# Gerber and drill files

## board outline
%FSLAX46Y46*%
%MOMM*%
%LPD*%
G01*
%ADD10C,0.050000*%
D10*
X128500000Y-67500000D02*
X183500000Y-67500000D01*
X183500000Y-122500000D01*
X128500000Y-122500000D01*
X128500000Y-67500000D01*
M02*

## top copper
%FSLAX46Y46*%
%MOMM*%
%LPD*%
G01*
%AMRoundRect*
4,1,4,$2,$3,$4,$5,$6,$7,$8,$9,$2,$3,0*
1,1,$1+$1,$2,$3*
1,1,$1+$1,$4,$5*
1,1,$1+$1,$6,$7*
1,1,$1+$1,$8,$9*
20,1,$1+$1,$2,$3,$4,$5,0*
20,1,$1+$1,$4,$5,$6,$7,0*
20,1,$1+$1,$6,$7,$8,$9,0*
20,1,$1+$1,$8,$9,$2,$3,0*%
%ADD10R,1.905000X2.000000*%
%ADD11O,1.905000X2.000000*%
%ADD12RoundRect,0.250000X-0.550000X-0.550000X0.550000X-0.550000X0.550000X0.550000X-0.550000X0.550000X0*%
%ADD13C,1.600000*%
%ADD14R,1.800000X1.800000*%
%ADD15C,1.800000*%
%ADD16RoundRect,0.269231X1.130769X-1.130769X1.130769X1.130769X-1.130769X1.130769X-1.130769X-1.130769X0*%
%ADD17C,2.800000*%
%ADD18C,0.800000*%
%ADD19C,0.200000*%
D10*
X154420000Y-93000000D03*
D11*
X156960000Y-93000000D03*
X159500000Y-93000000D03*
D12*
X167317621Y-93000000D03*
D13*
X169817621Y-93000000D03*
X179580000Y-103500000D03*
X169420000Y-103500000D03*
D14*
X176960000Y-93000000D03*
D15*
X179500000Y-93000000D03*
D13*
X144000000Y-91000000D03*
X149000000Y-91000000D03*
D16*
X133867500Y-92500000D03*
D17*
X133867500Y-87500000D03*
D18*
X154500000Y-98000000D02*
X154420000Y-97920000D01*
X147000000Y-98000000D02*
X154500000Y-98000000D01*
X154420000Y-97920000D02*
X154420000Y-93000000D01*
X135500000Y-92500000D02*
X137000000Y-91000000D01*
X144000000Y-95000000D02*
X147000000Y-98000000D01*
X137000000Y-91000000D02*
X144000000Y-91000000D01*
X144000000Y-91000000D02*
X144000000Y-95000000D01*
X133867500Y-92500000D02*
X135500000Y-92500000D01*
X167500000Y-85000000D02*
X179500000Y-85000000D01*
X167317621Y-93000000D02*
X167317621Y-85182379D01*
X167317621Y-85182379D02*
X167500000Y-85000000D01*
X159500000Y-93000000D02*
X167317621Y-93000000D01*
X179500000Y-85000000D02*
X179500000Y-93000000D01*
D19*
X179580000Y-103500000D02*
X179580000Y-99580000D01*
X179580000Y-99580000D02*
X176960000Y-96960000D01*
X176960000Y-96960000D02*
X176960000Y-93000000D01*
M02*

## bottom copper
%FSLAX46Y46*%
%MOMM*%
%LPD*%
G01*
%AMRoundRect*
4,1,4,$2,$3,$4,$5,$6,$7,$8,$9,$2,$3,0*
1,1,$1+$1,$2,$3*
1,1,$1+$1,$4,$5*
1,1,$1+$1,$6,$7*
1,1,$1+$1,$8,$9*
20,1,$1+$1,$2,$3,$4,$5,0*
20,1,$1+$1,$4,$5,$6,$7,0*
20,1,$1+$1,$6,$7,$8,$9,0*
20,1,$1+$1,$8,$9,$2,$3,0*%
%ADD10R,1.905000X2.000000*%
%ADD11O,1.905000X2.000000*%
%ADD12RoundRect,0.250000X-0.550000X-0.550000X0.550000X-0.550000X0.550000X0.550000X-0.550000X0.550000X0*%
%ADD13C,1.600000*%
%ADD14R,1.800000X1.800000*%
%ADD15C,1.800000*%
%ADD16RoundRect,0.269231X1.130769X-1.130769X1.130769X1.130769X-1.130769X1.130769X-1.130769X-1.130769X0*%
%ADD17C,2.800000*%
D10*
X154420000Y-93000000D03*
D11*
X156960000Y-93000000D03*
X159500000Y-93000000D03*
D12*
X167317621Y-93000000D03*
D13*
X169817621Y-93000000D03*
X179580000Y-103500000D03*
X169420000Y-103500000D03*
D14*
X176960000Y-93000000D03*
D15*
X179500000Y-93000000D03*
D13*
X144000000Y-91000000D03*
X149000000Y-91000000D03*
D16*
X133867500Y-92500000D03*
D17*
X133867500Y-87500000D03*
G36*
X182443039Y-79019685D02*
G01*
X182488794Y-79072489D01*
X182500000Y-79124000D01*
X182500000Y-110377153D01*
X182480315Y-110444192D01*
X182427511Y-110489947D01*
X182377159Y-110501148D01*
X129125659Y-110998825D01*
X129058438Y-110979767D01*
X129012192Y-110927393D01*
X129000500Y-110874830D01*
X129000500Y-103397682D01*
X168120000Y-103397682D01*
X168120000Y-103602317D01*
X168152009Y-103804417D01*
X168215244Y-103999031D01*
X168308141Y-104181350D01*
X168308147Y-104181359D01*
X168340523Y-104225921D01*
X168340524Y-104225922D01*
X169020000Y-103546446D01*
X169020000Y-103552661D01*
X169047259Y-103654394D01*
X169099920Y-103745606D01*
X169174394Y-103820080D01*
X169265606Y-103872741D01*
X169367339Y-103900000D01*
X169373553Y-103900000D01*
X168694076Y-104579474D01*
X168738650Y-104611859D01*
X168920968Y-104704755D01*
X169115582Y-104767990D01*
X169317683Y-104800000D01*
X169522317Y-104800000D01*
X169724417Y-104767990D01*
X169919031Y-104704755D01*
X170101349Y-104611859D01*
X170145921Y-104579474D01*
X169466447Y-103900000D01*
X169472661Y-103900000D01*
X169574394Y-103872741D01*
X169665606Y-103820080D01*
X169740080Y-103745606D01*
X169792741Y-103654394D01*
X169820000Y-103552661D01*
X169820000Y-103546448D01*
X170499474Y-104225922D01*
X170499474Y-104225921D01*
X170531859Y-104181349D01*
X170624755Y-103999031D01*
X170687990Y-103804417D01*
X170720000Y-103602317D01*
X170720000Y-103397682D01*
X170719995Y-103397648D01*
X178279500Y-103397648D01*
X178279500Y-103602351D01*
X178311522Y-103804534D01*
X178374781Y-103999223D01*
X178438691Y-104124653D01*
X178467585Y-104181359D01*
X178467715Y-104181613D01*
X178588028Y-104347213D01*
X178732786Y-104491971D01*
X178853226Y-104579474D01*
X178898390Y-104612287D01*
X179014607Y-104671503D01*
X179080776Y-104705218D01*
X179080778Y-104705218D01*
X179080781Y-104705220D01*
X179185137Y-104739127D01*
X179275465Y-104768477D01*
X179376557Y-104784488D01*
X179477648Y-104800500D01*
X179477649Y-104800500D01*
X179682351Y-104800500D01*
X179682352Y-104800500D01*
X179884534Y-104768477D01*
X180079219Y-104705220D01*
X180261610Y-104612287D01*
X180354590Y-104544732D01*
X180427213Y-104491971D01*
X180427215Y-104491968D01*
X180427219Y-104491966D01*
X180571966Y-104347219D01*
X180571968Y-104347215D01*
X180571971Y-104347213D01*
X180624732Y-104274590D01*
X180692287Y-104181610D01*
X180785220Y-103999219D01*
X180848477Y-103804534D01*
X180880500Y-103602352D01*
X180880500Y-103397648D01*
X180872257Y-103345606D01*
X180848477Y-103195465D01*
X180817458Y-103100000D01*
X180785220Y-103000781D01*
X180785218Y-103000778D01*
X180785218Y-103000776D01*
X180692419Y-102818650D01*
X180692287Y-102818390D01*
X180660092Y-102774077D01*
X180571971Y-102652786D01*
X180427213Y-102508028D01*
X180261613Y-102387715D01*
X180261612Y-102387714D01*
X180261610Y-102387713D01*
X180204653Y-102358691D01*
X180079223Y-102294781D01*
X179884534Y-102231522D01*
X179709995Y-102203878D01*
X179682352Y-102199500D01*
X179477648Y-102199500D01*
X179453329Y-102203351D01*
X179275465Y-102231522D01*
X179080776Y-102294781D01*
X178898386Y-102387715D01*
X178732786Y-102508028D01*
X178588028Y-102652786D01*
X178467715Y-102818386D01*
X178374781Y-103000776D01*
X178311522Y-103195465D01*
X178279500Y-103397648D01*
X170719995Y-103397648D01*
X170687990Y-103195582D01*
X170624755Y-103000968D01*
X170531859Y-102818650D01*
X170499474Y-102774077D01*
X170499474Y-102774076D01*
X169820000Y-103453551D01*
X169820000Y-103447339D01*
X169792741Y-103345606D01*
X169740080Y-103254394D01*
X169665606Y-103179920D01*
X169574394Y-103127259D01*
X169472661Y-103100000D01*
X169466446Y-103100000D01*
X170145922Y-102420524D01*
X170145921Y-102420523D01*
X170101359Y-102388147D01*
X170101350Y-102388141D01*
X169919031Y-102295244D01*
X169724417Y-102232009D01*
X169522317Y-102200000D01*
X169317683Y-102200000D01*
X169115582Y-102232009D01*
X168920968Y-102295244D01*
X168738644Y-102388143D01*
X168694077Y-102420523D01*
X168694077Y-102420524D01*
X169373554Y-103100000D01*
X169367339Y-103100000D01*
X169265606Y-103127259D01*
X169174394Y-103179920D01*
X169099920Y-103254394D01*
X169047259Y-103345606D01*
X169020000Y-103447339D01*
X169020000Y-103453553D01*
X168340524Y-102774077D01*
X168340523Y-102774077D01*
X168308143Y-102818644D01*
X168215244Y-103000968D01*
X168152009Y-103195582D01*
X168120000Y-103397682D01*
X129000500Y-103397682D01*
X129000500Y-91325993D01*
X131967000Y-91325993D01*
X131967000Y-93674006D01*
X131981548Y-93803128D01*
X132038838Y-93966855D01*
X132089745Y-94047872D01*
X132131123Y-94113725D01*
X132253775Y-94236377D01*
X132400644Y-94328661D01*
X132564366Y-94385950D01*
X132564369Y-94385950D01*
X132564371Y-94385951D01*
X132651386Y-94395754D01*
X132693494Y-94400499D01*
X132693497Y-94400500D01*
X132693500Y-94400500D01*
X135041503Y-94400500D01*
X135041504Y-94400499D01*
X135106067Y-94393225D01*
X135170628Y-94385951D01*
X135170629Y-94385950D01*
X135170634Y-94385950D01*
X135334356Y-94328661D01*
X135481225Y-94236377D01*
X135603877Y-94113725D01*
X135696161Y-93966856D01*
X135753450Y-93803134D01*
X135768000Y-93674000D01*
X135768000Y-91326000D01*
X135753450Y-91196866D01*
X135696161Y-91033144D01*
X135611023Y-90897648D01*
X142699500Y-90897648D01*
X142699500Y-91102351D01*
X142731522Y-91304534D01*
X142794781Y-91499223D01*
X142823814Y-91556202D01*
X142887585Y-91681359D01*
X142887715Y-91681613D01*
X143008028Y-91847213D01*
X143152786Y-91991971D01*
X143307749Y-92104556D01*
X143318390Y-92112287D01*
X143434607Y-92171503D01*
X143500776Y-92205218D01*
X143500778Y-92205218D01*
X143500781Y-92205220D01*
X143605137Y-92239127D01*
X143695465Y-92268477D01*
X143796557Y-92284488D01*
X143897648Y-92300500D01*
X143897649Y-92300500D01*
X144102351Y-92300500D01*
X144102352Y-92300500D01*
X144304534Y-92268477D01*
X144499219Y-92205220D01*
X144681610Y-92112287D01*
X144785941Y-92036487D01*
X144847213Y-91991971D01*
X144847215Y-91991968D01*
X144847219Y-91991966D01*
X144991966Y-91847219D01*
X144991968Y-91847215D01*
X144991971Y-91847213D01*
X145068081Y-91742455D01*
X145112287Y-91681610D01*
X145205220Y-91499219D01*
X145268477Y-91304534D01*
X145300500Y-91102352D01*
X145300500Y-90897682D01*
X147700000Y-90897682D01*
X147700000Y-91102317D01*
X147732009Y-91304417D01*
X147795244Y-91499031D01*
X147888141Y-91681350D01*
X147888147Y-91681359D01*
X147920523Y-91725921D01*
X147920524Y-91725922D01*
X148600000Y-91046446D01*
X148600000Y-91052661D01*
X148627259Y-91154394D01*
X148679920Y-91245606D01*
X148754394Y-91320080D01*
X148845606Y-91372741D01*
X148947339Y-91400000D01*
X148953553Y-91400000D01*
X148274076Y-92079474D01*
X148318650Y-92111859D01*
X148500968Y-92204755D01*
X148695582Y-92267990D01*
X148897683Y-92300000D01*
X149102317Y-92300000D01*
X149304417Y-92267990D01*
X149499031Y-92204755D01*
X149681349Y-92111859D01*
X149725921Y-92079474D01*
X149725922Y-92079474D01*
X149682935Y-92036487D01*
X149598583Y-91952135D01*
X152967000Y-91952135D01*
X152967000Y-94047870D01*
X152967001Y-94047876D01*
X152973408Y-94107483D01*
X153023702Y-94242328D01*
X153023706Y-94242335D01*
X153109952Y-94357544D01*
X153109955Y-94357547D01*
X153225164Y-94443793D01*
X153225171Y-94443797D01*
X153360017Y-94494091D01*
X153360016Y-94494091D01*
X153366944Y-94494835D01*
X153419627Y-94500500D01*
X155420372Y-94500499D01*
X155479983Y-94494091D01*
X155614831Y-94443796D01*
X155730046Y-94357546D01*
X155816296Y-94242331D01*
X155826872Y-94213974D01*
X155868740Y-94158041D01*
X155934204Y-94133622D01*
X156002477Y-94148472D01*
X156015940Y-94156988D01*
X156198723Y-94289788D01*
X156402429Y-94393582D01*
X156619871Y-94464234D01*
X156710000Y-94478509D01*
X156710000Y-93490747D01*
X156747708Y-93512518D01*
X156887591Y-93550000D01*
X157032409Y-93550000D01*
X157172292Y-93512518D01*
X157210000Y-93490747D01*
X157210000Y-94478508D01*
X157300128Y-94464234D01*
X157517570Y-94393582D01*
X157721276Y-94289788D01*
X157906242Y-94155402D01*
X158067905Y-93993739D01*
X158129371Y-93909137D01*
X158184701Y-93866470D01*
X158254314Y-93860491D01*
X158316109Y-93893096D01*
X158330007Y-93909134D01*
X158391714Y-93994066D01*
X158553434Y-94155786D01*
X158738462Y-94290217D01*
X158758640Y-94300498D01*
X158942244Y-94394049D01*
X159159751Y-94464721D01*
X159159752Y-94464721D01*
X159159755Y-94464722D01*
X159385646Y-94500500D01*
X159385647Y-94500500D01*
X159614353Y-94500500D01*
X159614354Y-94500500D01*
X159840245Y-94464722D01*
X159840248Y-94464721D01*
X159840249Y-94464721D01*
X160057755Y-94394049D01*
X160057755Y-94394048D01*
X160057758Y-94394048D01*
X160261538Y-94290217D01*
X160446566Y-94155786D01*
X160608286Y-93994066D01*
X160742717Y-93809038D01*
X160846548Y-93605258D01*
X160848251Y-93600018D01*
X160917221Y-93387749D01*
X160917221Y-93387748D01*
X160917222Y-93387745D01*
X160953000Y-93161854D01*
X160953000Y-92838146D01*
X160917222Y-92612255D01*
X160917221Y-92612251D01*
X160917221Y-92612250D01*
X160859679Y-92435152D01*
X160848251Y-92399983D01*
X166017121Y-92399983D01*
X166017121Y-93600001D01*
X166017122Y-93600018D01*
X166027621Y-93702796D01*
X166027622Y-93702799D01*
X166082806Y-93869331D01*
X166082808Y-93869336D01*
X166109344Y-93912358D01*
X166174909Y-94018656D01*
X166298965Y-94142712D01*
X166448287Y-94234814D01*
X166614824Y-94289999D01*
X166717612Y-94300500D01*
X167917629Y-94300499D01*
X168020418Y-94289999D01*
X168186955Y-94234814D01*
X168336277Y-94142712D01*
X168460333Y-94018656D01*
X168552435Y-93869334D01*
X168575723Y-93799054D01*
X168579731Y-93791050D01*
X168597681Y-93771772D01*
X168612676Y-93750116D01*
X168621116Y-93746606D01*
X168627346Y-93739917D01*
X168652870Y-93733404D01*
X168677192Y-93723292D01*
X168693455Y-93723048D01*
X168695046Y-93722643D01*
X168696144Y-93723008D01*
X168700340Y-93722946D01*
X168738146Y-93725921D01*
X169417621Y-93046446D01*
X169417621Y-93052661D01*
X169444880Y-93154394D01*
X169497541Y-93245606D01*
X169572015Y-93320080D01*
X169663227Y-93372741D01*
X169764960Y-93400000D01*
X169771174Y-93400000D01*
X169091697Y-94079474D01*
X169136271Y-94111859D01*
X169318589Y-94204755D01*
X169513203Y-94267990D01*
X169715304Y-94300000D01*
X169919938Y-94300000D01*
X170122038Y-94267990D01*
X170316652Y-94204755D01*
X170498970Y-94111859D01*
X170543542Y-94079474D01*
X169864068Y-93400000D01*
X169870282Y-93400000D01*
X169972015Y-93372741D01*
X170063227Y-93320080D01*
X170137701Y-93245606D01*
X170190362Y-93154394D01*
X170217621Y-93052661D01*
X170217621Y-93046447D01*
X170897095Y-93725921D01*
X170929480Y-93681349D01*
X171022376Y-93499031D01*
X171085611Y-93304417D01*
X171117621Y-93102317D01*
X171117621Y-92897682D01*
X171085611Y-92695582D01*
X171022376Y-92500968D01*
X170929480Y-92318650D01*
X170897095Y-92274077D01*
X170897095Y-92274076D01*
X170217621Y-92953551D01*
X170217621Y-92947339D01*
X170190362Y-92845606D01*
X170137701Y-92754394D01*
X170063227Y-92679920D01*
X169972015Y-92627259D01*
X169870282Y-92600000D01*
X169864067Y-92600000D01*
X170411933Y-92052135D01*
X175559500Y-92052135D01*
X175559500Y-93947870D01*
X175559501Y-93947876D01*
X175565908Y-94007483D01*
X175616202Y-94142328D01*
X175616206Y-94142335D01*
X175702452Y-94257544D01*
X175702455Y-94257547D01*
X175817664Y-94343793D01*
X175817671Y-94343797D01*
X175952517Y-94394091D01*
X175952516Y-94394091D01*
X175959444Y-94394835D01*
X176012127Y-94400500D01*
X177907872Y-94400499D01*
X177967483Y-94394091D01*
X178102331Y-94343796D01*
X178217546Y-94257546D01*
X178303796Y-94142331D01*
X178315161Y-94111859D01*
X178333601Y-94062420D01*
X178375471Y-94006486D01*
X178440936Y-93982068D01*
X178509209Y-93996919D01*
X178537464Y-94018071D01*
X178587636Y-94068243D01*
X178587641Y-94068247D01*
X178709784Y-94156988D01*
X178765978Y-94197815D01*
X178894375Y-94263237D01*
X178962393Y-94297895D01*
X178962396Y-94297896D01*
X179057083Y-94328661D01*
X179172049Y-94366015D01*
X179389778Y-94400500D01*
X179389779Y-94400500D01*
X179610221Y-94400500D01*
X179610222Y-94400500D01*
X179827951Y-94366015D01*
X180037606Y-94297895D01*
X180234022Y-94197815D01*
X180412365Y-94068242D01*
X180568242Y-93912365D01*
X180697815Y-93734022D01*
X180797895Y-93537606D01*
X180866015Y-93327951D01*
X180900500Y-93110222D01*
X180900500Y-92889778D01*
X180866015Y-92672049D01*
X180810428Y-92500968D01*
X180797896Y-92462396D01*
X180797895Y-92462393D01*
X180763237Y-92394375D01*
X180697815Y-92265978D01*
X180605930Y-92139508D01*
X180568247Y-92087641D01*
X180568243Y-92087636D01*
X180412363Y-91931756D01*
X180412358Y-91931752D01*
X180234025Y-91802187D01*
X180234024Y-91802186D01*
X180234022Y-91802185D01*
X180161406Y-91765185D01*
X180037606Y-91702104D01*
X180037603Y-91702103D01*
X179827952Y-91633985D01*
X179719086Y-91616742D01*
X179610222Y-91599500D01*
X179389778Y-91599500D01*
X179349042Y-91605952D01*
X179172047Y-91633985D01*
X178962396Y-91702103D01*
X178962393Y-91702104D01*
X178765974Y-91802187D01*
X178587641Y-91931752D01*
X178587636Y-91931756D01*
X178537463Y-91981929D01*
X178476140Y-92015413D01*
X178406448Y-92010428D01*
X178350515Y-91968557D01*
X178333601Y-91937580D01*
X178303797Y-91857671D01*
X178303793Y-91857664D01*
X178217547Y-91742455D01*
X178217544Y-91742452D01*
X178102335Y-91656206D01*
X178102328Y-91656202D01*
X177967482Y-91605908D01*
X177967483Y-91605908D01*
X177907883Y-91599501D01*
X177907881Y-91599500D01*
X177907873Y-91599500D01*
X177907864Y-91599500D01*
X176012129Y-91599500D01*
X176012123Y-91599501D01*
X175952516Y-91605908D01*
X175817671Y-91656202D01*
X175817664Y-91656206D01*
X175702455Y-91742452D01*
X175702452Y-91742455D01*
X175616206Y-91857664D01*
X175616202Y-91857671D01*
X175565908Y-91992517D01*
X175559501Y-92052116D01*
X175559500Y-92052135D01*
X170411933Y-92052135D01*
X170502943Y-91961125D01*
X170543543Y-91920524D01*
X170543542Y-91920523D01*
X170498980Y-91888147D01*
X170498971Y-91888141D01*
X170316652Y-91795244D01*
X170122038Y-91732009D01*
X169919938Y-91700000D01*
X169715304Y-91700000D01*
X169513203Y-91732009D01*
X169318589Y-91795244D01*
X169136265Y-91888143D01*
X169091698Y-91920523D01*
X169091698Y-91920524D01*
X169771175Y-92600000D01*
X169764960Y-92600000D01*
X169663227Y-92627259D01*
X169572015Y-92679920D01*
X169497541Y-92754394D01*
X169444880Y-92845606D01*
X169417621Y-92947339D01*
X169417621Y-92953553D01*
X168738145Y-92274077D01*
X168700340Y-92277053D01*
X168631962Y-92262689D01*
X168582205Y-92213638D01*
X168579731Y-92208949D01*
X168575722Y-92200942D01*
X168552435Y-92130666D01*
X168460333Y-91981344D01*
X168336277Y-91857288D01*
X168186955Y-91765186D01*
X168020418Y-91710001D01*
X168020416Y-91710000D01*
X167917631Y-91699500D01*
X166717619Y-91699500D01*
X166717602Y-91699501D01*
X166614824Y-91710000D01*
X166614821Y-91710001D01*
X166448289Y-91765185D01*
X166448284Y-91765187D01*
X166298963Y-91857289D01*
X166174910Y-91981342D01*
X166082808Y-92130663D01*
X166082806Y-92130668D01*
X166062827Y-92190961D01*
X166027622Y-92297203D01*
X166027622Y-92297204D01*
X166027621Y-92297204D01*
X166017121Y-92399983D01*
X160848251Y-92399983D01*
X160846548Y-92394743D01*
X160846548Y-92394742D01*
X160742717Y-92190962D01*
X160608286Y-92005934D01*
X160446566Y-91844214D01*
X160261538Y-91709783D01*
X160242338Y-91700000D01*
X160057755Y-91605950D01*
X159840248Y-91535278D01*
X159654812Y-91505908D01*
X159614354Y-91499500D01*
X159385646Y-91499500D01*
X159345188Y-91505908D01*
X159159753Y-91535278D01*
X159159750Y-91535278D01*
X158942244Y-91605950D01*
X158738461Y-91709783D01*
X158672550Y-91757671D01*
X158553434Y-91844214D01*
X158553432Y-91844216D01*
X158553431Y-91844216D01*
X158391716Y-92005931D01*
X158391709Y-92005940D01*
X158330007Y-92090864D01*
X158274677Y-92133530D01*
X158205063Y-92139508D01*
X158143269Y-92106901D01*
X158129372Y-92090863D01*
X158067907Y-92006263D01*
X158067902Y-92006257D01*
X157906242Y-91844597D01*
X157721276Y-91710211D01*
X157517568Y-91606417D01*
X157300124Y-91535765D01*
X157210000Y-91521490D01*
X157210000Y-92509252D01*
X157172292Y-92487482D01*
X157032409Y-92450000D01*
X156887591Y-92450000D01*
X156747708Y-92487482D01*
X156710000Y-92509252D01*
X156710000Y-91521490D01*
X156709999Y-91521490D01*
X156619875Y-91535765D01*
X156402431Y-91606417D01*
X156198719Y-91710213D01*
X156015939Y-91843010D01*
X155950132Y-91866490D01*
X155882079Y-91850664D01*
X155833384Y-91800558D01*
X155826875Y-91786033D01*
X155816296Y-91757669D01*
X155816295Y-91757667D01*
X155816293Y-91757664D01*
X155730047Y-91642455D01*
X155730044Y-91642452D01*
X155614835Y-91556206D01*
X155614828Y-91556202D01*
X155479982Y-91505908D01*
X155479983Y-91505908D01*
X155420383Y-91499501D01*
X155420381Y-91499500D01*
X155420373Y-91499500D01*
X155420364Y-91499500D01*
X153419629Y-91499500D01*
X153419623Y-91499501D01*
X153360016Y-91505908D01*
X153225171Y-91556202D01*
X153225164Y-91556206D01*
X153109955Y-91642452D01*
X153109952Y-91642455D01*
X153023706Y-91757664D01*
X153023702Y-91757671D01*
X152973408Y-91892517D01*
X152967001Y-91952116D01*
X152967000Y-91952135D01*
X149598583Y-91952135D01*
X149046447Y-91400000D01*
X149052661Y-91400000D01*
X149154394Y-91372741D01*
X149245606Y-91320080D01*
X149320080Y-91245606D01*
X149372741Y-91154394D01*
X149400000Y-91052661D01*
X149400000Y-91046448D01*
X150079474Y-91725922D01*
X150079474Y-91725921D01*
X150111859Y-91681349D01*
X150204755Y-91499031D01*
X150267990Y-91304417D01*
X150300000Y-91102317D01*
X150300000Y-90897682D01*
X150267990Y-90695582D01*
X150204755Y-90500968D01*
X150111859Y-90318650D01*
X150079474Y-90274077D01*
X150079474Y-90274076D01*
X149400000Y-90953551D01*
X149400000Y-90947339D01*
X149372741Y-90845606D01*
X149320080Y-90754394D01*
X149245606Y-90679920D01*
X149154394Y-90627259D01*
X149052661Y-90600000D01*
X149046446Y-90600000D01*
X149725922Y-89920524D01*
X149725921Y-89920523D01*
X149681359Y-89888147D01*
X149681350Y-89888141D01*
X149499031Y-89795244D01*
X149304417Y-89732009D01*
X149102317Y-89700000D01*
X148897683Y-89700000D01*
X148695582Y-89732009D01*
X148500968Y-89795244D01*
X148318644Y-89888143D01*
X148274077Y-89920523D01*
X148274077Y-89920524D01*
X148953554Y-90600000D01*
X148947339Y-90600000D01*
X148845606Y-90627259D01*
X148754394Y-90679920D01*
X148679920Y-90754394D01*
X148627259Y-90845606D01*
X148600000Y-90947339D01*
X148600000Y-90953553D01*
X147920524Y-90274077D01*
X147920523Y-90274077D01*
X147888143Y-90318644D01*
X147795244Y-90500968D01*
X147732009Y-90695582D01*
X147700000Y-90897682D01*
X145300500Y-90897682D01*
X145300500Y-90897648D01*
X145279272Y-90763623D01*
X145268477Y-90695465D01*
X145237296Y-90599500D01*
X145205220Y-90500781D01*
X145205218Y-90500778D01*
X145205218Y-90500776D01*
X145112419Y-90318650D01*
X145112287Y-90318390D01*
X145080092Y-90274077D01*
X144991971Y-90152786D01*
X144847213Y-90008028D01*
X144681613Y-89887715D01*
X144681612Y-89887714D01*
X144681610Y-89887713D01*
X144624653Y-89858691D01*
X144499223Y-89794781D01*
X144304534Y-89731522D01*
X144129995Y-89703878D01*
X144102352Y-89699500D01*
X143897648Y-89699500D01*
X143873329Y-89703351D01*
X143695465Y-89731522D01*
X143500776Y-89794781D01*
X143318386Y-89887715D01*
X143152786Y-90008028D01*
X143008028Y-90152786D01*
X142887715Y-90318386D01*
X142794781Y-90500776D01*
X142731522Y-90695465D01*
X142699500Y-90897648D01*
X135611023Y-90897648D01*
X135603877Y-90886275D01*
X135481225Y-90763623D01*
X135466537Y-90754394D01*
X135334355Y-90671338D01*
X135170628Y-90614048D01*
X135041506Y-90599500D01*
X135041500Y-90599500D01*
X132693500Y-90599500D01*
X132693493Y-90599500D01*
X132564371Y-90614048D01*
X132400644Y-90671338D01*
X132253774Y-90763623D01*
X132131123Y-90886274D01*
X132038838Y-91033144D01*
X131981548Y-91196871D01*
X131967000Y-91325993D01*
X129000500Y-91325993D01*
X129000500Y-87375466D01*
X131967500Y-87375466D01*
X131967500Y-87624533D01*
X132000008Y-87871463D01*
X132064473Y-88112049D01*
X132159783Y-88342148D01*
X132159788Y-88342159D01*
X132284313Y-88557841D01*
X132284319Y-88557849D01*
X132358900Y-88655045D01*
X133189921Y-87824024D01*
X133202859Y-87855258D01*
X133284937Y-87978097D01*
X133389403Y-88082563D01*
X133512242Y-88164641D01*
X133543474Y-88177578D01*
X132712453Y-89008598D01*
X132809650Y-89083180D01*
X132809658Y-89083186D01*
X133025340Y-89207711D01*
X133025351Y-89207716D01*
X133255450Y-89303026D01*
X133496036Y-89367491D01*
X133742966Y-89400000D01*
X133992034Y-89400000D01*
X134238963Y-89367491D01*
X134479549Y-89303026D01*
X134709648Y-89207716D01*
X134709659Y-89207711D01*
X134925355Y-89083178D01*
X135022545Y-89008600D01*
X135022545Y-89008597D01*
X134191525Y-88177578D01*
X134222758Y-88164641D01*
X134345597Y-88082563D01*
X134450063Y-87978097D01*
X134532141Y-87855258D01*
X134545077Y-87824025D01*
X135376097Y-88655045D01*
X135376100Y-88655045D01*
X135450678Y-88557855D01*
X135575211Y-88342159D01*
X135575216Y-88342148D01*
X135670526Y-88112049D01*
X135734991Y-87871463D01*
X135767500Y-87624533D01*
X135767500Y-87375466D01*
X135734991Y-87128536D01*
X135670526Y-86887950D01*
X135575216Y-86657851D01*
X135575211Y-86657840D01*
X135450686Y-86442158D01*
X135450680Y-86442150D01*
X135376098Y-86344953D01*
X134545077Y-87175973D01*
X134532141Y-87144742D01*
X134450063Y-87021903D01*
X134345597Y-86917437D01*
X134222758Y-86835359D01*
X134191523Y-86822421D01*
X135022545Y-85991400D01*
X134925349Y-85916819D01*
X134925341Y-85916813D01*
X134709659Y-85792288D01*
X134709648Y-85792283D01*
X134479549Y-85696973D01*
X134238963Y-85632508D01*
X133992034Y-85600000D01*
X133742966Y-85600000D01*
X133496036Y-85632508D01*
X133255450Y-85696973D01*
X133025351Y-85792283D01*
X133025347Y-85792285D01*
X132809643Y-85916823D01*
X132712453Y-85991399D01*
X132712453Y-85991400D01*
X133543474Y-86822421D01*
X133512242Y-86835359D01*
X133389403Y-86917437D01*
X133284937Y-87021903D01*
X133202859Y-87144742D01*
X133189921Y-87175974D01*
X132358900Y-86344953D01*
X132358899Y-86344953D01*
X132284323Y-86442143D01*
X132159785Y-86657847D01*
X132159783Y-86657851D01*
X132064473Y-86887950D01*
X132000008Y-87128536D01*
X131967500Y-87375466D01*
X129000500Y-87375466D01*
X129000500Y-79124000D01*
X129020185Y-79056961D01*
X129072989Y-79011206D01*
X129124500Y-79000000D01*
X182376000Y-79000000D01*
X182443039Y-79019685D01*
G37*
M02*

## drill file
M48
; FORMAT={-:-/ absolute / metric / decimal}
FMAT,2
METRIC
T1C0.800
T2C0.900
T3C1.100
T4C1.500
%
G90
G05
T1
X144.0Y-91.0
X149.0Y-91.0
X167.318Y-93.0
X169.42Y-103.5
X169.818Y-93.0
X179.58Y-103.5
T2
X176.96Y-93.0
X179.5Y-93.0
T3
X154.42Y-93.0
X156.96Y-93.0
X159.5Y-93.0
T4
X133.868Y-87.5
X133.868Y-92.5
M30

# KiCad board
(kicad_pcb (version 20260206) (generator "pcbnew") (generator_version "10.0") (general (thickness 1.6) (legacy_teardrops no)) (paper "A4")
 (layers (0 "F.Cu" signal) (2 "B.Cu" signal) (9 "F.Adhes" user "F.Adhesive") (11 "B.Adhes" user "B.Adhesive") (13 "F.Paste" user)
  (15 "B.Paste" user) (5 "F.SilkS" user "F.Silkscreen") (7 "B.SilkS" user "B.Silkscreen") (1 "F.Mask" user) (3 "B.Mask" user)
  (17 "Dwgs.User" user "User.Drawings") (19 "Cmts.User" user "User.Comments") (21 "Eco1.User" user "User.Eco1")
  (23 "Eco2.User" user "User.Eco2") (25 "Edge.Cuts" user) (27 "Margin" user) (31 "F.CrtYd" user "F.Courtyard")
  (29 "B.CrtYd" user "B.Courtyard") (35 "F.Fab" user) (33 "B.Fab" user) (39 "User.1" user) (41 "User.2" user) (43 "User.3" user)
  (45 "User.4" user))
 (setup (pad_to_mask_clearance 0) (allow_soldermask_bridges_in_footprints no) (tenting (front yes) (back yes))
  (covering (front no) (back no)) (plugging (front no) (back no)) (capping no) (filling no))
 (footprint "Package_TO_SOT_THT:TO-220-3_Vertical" (layer "F.Cu") (at 154.42 93)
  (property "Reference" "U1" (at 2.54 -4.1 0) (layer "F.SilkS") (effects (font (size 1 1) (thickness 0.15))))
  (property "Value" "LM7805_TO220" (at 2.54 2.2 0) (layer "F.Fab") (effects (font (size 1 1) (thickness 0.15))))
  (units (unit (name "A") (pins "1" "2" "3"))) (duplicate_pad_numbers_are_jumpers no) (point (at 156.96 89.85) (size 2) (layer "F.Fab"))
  (pad "1" thru_hole rect (at 0 0) (size 1.905 2) (drill 1.1) (layers "*.Cu" "*.Mask") (remove_unused_layers no) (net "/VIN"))
  (pad "2" thru_hole oval (at 2.54 0) (size 1.905 2) (drill 1.1) (layers "*.Cu" "*.Mask") (remove_unused_layers no) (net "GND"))
  (pad "3" thru_hole oval (at 5.08 0) (size 1.905 2) (drill 1.1) (layers "*.Cu" "*.Mask") (remove_unused_layers no) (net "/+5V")))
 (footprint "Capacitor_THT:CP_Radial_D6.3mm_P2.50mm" (layer "F.Cu") (at 167.317621 93)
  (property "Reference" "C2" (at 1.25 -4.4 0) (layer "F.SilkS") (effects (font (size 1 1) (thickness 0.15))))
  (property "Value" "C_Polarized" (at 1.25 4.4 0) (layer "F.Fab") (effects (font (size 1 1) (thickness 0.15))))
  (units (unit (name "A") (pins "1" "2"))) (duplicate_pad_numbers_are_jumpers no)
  (pad "1" thru_hole roundrect (at 0 0) (size 1.6 1.6) (drill 0.8) (layers "*.Cu" "*.Mask") (remove_unused_layers no)
   (roundrect_rratio 0.15625) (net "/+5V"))
  (pad "2" thru_hole circle (at 2.5 0) (size 1.6 1.6) (drill 0.8) (layers "*.Cu" "*.Mask") (remove_unused_layers no) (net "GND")))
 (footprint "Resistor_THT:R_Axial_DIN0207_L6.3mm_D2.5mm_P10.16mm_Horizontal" (layer "F.Cu") (at 179.58 103.5 180)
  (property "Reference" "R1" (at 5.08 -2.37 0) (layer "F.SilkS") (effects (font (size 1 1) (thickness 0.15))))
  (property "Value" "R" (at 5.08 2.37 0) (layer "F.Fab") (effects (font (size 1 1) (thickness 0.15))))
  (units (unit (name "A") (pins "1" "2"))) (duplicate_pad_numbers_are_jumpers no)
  (pad "1" thru_hole circle (at 0 0 180) (size 1.6 1.6) (drill 0.8) (layers "*.Cu" "*.Mask") (remove_unused_layers no) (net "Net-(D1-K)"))
  (pad "2" thru_hole circle (at 10.16 0 180) (size 1.6 1.6) (drill 0.8) (layers "*.Cu" "*.Mask") (remove_unused_layers no) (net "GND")))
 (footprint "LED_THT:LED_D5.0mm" (layer "F.Cu") (at 176.96 93)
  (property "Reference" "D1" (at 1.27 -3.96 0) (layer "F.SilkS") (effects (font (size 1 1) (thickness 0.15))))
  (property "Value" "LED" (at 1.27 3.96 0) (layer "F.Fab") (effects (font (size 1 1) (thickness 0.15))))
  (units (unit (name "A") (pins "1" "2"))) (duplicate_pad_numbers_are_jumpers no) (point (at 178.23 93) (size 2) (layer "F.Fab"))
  (pad "1" thru_hole rect (at 0 0) (size 1.8 1.8) (drill 0.9) (layers "*.Cu" "*.Mask") (remove_unused_layers no) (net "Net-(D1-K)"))
  (pad "2" thru_hole circle (at 2.54 0) (size 1.8 1.8) (drill 0.9) (layers "*.Cu" "*.Mask") (remove_unused_layers no) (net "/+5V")))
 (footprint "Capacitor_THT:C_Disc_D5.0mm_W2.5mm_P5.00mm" (layer "F.Cu") (at 144 91)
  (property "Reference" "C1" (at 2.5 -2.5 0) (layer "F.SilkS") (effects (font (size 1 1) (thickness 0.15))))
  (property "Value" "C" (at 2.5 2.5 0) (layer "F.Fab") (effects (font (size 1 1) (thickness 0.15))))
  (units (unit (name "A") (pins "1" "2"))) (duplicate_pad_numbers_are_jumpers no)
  (pad "1" thru_hole circle (at 0 0) (size 1.6 1.6) (drill 0.8) (layers "*.Cu" "*.Mask") (remove_unused_layers no) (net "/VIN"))
  (pad "2" thru_hole circle (at 5 0) (size 1.6 1.6) (drill 0.8) (layers "*.Cu" "*.Mask") (remove_unused_layers no) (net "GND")))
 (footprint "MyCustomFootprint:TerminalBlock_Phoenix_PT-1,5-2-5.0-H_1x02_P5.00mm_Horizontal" (layer "F.Cu") (at 133.8675 92.5 90)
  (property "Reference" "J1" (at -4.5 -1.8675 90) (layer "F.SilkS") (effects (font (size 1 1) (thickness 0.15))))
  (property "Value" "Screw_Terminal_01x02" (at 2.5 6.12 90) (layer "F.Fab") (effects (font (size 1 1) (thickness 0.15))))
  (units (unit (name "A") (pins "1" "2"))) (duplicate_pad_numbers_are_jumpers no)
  (pad "1" thru_hole roundrect (at 0 0 90) (size 2.8 2.8) (drill 1.5) (layers "*.Cu" "*.Mask") (remove_unused_layers no)
   (roundrect_rratio 0.096154) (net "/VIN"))
  (pad "2" thru_hole circle (at 5 0 90) (size 2.8 2.8) (drill 1.5) (layers "*.Cu" "*.Mask") (remove_unused_layers no) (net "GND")))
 (gr_rect (start 128.5 67.5) (end 183.5 122.5) (stroke (width 0.05) (type default)) (fill no) (layer "Edge.Cuts"))
 (segment (start 154.5 98) (end 154.42 97.92) (width 0.8) (layer "F.Cu") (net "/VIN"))
 (segment (start 147 98) (end 154.5 98) (width 0.8) (layer "F.Cu") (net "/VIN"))
 (segment (start 154.42 97.92) (end 154.42 93) (width 0.8) (layer "F.Cu") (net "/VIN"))
 (segment (start 135.5 92.5) (end 137 91) (width 0.8) (layer "F.Cu") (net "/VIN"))
 (segment (start 144 95) (end 147 98) (width 0.8) (layer "F.Cu") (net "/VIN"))
 (segment (start 137 91) (end 144 91) (width 0.8) (layer "F.Cu") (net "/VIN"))
 (segment (start 144 91) (end 144 95) (width 0.8) (layer "F.Cu") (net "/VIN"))
 (segment (start 133.8675 92.5) (end 135.5 92.5) (width 0.8) (layer "F.Cu") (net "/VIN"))
 (segment (start 167.5 85) (end 179.5 85) (width 0.8) (layer "F.Cu") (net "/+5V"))
 (segment (start 167.317621 93) (end 167.317621 85.182379) (width 0.8) (layer "F.Cu") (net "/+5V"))
 (segment (start 167.317621 85.182379) (end 167.5 85) (width 0.8) (layer "F.Cu") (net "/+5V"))
 (segment (start 159.5 93) (end 167.317621 93) (width 0.8) (layer "F.Cu") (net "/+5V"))
 (segment (start 179.5 85) (end 179.5 93) (width 0.8) (layer "F.Cu") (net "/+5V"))
 (segment (start 179.58 103.5) (end 179.58 99.58) (width 0.2) (layer "F.Cu") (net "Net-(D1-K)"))
 (segment (start 179.58 99.58) (end 176.96 96.96) (width 0.2) (layer "F.Cu") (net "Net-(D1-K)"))
 (segment (start 176.96 96.96) (end 176.96 93) (width 0.2) (layer "F.Cu") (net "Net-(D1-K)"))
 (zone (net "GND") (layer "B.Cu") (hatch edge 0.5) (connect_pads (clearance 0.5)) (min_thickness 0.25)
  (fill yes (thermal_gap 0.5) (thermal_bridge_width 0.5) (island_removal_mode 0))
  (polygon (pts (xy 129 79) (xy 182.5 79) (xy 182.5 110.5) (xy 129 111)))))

